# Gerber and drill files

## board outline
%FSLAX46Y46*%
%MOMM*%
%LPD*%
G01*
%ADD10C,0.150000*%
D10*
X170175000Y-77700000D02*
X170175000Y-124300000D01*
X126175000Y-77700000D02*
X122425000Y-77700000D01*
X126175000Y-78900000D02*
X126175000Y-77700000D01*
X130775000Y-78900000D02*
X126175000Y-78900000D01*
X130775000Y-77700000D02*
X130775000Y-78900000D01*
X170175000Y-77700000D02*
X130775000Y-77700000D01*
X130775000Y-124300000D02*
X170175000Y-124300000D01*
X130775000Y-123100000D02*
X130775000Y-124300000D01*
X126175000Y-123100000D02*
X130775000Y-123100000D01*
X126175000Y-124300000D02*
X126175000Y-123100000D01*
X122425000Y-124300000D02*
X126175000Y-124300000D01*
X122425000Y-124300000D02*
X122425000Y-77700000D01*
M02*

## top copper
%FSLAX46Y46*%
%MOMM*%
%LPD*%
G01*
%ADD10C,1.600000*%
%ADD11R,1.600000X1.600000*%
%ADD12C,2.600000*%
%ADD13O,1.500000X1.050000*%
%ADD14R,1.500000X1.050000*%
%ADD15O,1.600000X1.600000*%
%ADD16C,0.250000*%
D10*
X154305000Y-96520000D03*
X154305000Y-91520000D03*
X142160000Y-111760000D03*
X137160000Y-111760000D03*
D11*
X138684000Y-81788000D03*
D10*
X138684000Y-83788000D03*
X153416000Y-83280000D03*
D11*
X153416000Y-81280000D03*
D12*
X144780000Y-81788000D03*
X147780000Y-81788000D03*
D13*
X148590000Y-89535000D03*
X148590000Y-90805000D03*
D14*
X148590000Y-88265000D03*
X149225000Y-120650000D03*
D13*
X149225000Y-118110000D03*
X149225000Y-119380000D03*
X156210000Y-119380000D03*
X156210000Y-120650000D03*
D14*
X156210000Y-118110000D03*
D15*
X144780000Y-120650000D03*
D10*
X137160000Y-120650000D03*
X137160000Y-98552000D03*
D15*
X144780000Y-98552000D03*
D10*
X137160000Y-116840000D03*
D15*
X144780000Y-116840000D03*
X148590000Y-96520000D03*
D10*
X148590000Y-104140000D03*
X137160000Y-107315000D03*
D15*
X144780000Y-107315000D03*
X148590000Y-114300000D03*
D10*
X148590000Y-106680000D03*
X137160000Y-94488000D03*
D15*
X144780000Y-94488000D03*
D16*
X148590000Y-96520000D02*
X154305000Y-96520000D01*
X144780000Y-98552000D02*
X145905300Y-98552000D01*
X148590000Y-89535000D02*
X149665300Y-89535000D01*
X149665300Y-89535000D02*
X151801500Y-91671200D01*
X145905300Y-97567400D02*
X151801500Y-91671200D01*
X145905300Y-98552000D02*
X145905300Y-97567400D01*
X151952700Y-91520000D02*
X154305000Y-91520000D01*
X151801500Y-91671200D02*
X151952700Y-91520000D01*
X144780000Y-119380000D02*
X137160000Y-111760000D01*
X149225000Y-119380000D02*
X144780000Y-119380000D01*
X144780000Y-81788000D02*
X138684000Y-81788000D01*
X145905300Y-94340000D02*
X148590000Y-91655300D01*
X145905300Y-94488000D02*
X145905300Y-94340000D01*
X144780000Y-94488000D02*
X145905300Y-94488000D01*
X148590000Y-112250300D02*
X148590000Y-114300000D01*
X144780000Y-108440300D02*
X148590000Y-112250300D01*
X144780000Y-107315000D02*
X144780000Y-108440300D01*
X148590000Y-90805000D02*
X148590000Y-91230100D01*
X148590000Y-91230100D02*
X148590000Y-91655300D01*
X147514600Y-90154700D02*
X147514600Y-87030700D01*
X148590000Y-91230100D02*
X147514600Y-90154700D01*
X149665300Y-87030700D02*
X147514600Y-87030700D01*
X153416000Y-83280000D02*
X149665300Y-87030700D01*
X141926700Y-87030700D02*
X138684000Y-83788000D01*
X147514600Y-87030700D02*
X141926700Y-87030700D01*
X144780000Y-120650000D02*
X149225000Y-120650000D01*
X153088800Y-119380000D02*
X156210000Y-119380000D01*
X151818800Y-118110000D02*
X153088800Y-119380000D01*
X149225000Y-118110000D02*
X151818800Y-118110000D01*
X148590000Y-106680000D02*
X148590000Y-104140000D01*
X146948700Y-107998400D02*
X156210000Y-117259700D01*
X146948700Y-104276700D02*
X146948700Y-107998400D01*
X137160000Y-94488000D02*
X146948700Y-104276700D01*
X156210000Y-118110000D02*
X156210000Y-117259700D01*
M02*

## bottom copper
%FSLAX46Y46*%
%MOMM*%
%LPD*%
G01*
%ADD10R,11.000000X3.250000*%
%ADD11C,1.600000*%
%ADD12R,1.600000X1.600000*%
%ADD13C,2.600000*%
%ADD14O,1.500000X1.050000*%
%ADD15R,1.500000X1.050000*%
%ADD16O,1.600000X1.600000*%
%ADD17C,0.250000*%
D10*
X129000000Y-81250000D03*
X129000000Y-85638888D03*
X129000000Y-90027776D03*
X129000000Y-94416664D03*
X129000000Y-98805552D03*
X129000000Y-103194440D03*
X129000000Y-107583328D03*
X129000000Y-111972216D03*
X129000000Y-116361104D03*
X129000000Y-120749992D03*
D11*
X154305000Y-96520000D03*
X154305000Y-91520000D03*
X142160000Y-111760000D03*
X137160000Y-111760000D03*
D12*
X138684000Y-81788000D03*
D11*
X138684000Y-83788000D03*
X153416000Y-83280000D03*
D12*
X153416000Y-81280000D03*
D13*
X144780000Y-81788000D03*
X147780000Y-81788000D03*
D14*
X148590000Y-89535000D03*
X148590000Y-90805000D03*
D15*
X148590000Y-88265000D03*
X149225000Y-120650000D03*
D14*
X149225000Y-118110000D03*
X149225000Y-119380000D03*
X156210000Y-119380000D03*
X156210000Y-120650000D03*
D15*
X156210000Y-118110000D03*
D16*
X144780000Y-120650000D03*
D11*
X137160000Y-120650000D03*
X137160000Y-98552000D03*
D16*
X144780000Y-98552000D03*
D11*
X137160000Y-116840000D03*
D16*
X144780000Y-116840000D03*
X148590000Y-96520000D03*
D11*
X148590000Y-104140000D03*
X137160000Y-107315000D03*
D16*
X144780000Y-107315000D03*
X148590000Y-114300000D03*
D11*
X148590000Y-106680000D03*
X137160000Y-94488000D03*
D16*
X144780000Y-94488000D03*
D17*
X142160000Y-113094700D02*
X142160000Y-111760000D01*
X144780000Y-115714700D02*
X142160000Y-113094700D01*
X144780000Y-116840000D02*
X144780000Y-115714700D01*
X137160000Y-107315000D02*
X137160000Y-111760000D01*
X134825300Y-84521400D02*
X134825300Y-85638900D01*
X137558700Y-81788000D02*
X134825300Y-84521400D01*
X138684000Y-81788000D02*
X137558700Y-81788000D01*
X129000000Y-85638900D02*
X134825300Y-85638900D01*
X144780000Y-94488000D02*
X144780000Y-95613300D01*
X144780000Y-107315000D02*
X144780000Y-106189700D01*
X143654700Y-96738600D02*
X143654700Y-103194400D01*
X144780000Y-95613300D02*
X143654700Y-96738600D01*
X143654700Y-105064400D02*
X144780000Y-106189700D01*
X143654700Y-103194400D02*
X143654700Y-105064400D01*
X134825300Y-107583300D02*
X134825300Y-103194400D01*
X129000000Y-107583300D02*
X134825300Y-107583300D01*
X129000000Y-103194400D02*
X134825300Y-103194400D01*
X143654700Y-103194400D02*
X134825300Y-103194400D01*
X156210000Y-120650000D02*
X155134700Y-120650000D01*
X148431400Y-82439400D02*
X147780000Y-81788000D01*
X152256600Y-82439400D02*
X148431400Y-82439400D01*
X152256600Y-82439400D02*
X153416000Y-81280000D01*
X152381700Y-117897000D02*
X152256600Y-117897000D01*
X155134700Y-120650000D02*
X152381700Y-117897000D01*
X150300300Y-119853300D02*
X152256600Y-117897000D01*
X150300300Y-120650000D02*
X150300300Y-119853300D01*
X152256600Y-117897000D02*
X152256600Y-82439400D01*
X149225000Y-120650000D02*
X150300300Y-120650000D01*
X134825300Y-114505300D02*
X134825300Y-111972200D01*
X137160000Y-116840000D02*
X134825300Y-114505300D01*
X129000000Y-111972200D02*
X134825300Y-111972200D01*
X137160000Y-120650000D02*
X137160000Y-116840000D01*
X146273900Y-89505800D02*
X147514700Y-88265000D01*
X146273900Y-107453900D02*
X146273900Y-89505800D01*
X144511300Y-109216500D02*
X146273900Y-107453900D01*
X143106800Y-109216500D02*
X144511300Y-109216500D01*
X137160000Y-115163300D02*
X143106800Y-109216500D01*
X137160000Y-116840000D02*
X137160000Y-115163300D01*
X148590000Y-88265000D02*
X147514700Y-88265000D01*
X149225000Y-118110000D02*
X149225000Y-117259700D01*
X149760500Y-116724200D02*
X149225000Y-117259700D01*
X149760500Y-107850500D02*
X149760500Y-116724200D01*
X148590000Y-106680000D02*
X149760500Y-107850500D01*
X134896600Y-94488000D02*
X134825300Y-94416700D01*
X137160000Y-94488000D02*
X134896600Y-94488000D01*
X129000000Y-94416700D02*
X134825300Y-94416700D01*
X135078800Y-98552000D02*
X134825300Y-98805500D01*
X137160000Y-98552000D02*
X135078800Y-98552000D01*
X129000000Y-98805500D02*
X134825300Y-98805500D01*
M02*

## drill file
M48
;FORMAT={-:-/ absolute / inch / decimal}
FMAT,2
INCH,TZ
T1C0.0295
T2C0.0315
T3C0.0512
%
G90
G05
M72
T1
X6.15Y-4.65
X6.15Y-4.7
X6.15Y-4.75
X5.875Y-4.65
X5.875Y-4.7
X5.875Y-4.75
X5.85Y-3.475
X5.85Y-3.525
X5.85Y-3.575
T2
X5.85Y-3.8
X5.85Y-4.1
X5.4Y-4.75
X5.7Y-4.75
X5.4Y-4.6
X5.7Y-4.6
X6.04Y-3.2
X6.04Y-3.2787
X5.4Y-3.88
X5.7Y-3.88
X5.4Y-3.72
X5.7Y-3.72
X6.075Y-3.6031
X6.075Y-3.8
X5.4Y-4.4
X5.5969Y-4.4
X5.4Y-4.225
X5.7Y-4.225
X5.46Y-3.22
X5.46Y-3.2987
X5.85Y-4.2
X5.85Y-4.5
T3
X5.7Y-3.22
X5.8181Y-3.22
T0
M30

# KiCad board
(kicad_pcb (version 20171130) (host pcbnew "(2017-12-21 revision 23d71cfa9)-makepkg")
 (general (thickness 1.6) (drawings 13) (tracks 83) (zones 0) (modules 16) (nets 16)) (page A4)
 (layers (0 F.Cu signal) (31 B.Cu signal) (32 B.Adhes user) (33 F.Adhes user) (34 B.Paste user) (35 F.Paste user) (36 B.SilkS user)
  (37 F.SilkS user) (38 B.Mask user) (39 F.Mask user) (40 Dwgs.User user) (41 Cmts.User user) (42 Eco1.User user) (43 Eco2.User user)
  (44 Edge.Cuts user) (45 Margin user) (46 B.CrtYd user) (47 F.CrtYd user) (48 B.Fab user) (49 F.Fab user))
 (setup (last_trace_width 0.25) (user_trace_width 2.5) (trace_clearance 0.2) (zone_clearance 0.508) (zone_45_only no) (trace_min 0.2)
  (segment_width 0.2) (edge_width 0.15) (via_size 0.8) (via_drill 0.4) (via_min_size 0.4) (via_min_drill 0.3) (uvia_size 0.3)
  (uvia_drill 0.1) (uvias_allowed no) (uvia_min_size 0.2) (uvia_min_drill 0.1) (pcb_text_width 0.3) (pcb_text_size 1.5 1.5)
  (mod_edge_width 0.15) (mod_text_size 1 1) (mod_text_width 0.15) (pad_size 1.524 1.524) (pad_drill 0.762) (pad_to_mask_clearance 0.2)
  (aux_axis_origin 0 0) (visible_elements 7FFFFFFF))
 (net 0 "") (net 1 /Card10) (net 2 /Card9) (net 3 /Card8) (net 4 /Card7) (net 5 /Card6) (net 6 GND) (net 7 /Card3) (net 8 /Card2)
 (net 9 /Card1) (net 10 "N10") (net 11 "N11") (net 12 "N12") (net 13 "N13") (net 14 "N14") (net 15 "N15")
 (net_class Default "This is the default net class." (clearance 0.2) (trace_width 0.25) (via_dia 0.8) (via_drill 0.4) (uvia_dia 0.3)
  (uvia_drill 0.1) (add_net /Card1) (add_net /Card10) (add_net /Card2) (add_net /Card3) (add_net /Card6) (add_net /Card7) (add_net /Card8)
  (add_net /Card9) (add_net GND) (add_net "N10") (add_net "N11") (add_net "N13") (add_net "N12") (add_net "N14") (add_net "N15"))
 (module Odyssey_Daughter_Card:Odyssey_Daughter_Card (layer F.Cu) (at 129 101)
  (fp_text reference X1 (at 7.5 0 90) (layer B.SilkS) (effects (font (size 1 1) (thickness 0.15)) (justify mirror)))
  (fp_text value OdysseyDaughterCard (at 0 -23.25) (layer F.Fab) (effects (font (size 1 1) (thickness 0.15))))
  (pad 10 smd rect (at 0 -19.75) (size 11 3.25) (layers B.Cu B.Mask) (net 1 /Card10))
  (pad 9 smd rect (at 0 -15.361112) (size 11 3.25) (layers B.Cu B.Mask) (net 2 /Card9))
  (pad 8 smd rect (at 0 -10.972224) (size 11 3.25) (layers B.Cu B.Mask) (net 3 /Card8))
  (pad 7 smd rect (at 0 -6.583336) (size 11 3.25) (layers B.Cu B.Mask) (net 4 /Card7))
  (pad 6 smd rect (at 0 -2.194448) (size 11 3.25) (layers B.Cu B.Mask) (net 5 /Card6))
  (pad 5 smd rect (at 0 2.19444) (size 11 3.25) (layers B.Cu B.Mask) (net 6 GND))
  (pad 4 smd rect (at 0 6.583328) (size 11 3.25) (layers B.Cu B.Mask) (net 6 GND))
  (pad 3 smd rect (at 0 10.972216) (size 11 3.25) (layers B.Cu B.Mask) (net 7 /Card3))
  (pad 2 smd rect (at 0 15.361104) (size 11 3.25) (layers B.Cu B.Mask) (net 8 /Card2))
  (pad 1 smd rect (at 0 19.749992) (size 11 3.25) (layers B.Cu B.Mask) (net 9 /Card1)))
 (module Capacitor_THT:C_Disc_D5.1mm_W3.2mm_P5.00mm (layer F.Cu) (at 154.305 96.52 90)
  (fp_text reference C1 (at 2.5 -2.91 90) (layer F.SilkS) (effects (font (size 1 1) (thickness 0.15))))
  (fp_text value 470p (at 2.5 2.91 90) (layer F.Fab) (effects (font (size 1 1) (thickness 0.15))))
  (pad 1 thru_hole circle (at 0 0 90) (size 1.6 1.6) (drill 0.8) (layers *.Cu *.Mask) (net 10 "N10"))
  (pad 2 thru_hole circle (at 5 0 90) (size 1.6 1.6) (drill 0.8) (layers *.Cu *.Mask) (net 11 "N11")))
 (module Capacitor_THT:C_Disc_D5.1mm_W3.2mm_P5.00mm (layer F.Cu) (at 137.16 111.76)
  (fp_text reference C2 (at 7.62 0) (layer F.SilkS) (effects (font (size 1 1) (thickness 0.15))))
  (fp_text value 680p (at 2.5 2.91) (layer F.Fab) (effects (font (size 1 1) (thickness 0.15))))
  (pad 2 thru_hole circle (at 5 0) (size 1.6 1.6) (drill 0.8) (layers *.Cu *.Mask) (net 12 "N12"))
  (pad 1 thru_hole circle (at 0 0) (size 1.6 1.6) (drill 0.8) (layers *.Cu *.Mask) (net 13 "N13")))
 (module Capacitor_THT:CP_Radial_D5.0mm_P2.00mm (layer F.Cu) (at 138.684 81.788 270)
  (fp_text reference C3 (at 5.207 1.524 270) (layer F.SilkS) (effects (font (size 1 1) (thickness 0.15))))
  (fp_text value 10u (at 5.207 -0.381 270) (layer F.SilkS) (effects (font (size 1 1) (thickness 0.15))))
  (pad 1 thru_hole rect (at 0 0 270) (size 1.6 1.6) (drill 0.8) (layers *.Cu *.Mask) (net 2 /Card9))
  (pad 2 thru_hole circle (at 2 0 270) (size 1.6 1.6) (drill 0.8) (layers *.Cu *.Mask) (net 6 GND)))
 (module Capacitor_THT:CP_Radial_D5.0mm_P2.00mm (layer F.Cu) (at 153.416 81.28 270)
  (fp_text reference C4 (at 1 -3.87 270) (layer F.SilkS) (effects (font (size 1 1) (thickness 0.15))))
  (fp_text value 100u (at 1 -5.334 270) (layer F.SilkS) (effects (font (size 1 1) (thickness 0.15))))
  (pad 2 thru_hole circle (at 2 0 270) (size 1.6 1.6) (drill 0.8) (layers *.Cu *.Mask) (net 6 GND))
  (pad 1 thru_hole rect (at 0 0 270) (size 1.6 1.6) (drill 0.8) (layers *.Cu *.Mask) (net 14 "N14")))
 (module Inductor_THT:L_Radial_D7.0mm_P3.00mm (layer F.Cu) (at 144.78 81.788)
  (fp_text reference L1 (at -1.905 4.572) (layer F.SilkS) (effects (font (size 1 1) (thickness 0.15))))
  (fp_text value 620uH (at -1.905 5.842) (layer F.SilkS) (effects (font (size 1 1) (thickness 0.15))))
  (pad 1 thru_hole circle (at 0 0) (size 2.6 2.6) (drill 1.3) (layers *.Cu *.Mask) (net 2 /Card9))
  (pad 2 thru_hole circle (at 3 0) (size 2.6 2.6) (drill 1.3) (layers *.Cu *.Mask) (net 14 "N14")))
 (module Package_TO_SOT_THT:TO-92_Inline (layer F.Cu) (at 148.59 88.265 270)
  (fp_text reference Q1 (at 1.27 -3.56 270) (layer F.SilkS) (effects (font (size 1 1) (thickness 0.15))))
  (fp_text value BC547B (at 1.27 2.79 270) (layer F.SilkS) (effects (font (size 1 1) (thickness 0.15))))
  (pad 2 thru_hole oval (at 1.27 0 270) (size 1.05 1.5) (drill 0.75) (layers *.Cu *.Mask) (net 11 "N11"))
  (pad 3 thru_hole oval (at 2.54 0 270) (size 1.05 1.5) (drill 0.75) (layers *.Cu *.Mask) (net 6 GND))
  (pad 1 thru_hole rect (at 0 0 270) (size 1.05 1.5) (drill 0.75) (layers *.Cu *.Mask) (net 7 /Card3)))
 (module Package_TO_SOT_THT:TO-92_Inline (layer F.Cu) (at 149.225 120.65 90)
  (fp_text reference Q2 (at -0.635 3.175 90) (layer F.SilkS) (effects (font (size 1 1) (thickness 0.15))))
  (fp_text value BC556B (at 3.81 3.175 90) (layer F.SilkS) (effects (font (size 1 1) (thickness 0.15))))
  (pad 1 thru_hole rect (at 0 0 90) (size 1.05 1.5) (drill 0.75) (layers *.Cu *.Mask) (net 14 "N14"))
  (pad 3 thru_hole oval (at 2.54 0 90) (size 1.05 1.5) (drill 0.75) (layers *.Cu *.Mask) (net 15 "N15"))
  (pad 2 thru_hole oval (at 1.27 0 90) (size 1.05 1.5) (drill 0.75) (layers *.Cu *.Mask) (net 13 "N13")))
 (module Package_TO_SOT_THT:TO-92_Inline (layer F.Cu) (at 156.21 118.11 270)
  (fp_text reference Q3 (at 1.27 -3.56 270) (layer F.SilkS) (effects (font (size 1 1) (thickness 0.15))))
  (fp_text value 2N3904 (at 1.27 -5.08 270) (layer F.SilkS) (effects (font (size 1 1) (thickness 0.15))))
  (pad 2 thru_hole oval (at 1.27 0 270) (size 1.05 1.5) (drill 0.75) (layers *.Cu *.Mask) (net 15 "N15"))
  (pad 3 thru_hole oval (at 2.54 0 270) (size 1.05 1.5) (drill 0.75) (layers *.Cu *.Mask) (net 14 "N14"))
  (pad 1 thru_hole rect (at 0 0 270) (size 1.05 1.5) (drill 0.75) (layers *.Cu *.Mask) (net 4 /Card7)))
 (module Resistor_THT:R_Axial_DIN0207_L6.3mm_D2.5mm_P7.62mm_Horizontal (layer F.Cu) (at 137.16 120.65)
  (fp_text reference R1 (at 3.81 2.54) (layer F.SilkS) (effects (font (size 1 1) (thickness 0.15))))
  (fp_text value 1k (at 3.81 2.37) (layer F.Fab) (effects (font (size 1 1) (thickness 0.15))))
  (pad 2 thru_hole oval (at 7.62 0) (size 1.6 1.6) (drill 0.8) (layers *.Cu *.Mask) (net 14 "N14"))
  (pad 1 thru_hole circle (at 0 0) (size 1.6 1.6) (drill 0.8) (layers *.Cu *.Mask) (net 7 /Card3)))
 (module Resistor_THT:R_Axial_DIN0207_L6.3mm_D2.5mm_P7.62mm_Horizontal (layer F.Cu) (at 137.16 98.552)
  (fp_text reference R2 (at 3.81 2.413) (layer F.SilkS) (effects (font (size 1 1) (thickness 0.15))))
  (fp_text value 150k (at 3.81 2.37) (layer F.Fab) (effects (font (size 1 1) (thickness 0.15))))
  (pad 1 thru_hole circle (at 0 0) (size 1.6 1.6) (drill 0.8) (layers *.Cu *.Mask) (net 5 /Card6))
  (pad 2 thru_hole oval (at 7.62 0) (size 1.6 1.6) (drill 0.8) (layers *.Cu *.Mask) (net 11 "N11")))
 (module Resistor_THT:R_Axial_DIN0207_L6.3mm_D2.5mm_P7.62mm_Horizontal (layer F.Cu) (at 137.16 116.84)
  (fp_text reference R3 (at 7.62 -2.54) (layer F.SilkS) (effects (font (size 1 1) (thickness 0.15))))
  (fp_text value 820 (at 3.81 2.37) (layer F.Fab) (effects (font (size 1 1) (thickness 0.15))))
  (pad 1 thru_hole circle (at 0 0) (size 1.6 1.6) (drill 0.8) (layers *.Cu *.Mask) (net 7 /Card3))
  (pad 2 thru_hole oval (at 7.62 0) (size 1.6 1.6) (drill 0.8) (layers *.Cu *.Mask) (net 12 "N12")))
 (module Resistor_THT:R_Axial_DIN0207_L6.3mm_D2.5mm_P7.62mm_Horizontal (layer F.Cu) (at 148.59 104.14 90)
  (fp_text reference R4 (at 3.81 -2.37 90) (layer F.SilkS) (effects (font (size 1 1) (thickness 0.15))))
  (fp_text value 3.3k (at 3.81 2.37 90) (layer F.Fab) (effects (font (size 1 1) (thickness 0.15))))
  (pad 2 thru_hole oval (at 7.62 0 90) (size 1.6 1.6) (drill 0.8) (layers *.Cu *.Mask) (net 10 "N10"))
  (pad 1 thru_hole circle (at 0 0 90) (size 1.6 1.6) (drill 0.8) (layers *.Cu *.Mask) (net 15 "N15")))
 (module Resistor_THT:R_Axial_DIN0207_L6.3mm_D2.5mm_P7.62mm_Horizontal (layer F.Cu) (at 137.16 107.315)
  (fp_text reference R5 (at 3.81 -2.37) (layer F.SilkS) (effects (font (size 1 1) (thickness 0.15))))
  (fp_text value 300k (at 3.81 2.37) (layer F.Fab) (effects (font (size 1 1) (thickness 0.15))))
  (pad 1 thru_hole circle (at 0 0) (size 1.6 1.6) (drill 0.8) (layers *.Cu *.Mask) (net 13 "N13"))
  (pad 2 thru_hole oval (at 7.62 0) (size 1.6 1.6) (drill 0.8) (layers *.Cu *.Mask) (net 6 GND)))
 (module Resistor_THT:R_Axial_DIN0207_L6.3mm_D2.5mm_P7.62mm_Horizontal (layer F.Cu) (at 148.59 106.68 270)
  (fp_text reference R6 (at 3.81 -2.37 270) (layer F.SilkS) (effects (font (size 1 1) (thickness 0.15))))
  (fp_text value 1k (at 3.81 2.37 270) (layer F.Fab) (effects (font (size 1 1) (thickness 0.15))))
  (pad 2 thru_hole oval (at 7.62 0 270) (size 1.6 1.6) (drill 0.8) (layers *.Cu *.Mask) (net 6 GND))
  (pad 1 thru_hole circle (at 0 0 270) (size 1.6 1.6) (drill 0.8) (layers *.Cu *.Mask) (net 15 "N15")))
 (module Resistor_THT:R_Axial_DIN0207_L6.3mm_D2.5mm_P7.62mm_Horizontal (layer F.Cu) (at 137.16 94.488)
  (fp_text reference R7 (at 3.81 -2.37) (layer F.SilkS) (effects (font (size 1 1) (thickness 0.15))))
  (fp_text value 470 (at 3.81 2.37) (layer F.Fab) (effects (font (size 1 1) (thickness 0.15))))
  (pad 1 thru_hole circle (at 0 0) (size 1.6 1.6) (drill 0.8) (layers *.Cu *.Mask) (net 4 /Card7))
  (pad 2 thru_hole oval (at 7.62 0) (size 1.6 1.6) (drill 0.8) (layers *.Cu *.Mask) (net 6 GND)))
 (gr_line (start 170.175 77.7) (end 170.175 124.3) (layer Edge.Cuts) (width 0.15))
 (gr_line (start 126.175 77.7) (end 122.425 77.7) (layer Edge.Cuts) (width 0.15))
 (gr_line (start 126.175 78.9) (end 126.175 77.7) (layer Edge.Cuts) (width 0.15))
 (gr_line (start 130.775 78.9) (end 126.175 78.9) (layer Edge.Cuts) (width 0.15))
 (gr_line (start 130.775 77.7) (end 130.775 78.9) (layer Edge.Cuts) (width 0.15))
 (gr_line (start 170.175 77.7) (end 130.775 77.7) (layer Edge.Cuts) (width 0.15))
 (gr_line (start 130.775 124.3) (end 170.175 124.3) (layer Edge.Cuts) (width 0.15))
 (gr_line (start 130.775 123.1) (end 130.775 124.3) (layer Edge.Cuts) (width 0.15))
 (gr_line (start 126.175 123.1) (end 130.775 123.1) (layer Edge.Cuts) (width 0.15))
 (gr_line (start 126.175 124.3) (end 126.175 123.1) (layer Edge.Cuts) (width 0.15))
 (gr_line (start 122.425 124.3) (end 126.175 124.3) (layer Edge.Cuts) (width 0.15))
 (gr_line (start 122.425 124.3) (end 122.425 77.7) (layer Edge.Cuts) (width 0.15))
 (segment (start 148.59 96.52) (end 154.305 96.52) (width 0.25) (layer F.Cu) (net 10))
 (segment (start 144.78 98.552) (end 145.9053 98.552) (width 0.25) (layer F.Cu) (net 11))
 (segment (start 148.59 89.535) (end 149.6653 89.535) (width 0.25) (layer F.Cu) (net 11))
 (segment (start 149.6653 89.535) (end 151.8015 91.6712) (width 0.25) (layer F.Cu) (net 11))
 (segment (start 145.9053 97.5674) (end 151.8015 91.6712) (width 0.25) (layer F.Cu) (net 11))
 (segment (start 145.9053 98.552) (end 145.9053 97.5674) (width 0.25) (layer F.Cu) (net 11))
 (segment (start 151.9527 91.52) (end 154.305 91.52) (width 0.25) (layer F.Cu) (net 11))
 (segment (start 151.8015 91.6712) (end 151.9527 91.52) (width 0.25) (layer F.Cu) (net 11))
 (segment (start 142.16 113.0947) (end 142.16 111.76) (width 0.25) (layer B.Cu) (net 12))
 (segment (start 144.78 115.7147) (end 142.16 113.0947) (width 0.25) (layer B.Cu) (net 12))
 (segment (start 144.78 116.84) (end 144.78 115.7147) (width 0.25) (layer B.Cu) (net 12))
 (segment (start 137.16 107.315) (end 137.16 111.76) (width 0.25) (layer B.Cu) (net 13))
 (segment (start 144.78 119.38) (end 137.16 111.76) (width 0.25) (layer F.Cu) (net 13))
 (segment (start 149.225 119.38) (end 144.78 119.38) (width 0.25) (layer F.Cu) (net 13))
 (segment (start 144.78 81.788) (end 138.684 81.788) (width 0.25) (layer F.Cu) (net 2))
 (segment (start 134.8253 84.5214) (end 134.8253 85.6389) (width 0.25) (layer B.Cu) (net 2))
 (segment (start 137.5587 81.788) (end 134.8253 84.5214) (width 0.25) (layer B.Cu) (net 2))
 (segment (start 138.684 81.788) (end 137.5587 81.788) (width 0.25) (layer B.Cu) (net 2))
 (segment (start 129 85.6389) (end 134.8253 85.6389) (width 0.25) (layer B.Cu) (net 2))
 (segment (start 145.9053 94.34) (end 148.59 91.6553) (width 0.25) (layer F.Cu) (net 6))
 (segment (start 145.9053 94.488) (end 145.9053 94.34) (width 0.25) (layer F.Cu) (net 6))
 (segment (start 144.78 94.488) (end 145.9053 94.488) (width 0.25) (layer F.Cu) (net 6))
 (segment (start 148.59 112.2503) (end 148.59 114.3) (width 0.25) (layer F.Cu) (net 6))
 (segment (start 144.78 108.4403) (end 148.59 112.2503) (width 0.25) (layer F.Cu) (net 6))
 (segment (start 144.78 107.315) (end 144.78 108.4403) (width 0.25) (layer F.Cu) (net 6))
 (segment (start 144.78 94.488) (end 144.78 95.6133) (width 0.25) (layer B.Cu) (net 6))
 (segment (start 144.78 107.315) (end 144.78 106.1897) (width 0.25) (layer B.Cu) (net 6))
 (segment (start 143.6547 96.7386) (end 143.6547 103.1944) (width 0.25) (layer B.Cu) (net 6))
 (segment (start 144.78 95.6133) (end 143.6547 96.7386) (width 0.25) (layer B.Cu) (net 6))
 (segment (start 143.6547 105.0644) (end 144.78 106.1897) (width 0.25) (layer B.Cu) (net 6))
 (segment (start 143.6547 103.1944) (end 143.6547 105.0644) (width 0.25) (layer B.Cu) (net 6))
 (segment (start 134.8253 107.5833) (end 134.8253 103.1944) (width 0.25) (layer B.Cu) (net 6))
 (segment (start 129 107.5833) (end 134.8253 107.5833) (width 0.25) (layer B.Cu) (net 6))
 (segment (start 129 103.1944) (end 134.8253 103.1944) (width 0.25) (layer B.Cu) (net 6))
 (segment (start 143.6547 103.1944) (end 134.8253 103.1944) (width 0.25) (layer B.Cu) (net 6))
 (segment (start 148.59 90.805) (end 148.59 91.2301) (width 0.25) (layer F.Cu) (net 6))
 (segment (start 148.59 91.2301) (end 148.59 91.6553) (width 0.25) (layer F.Cu) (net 6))
 (segment (start 147.5146 90.1547) (end 147.5146 87.0307) (width 0.25) (layer F.Cu) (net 6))
 (segment (start 148.59 91.2301) (end 147.5146 90.1547) (width 0.25) (layer F.Cu) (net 6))
 (segment (start 149.6653 87.0307) (end 147.5146 87.0307) (width 0.25) (layer F.Cu) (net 6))
 (segment (start 153.416 83.28) (end 149.6653 87.0307) (width 0.25) (layer F.Cu) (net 6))
 (segment (start 141.9267 87.0307) (end 138.684 83.788) (width 0.25) (layer F.Cu) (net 6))
 (segment (start 147.5146 87.0307) (end 141.9267 87.0307) (width 0.25) (layer F.Cu) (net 6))
 (segment (start 144.78 120.65) (end 149.225 120.65) (width 0.25) (layer F.Cu) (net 14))
 (segment (start 156.21 120.65) (end 155.1347 120.65) (width 0.25) (layer B.Cu) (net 14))
 (segment (start 148.4314 82.4394) (end 147.78 81.788) (width 0.25) (layer B.Cu) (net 14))
 (segment (start 152.2566 82.4394) (end 148.4314 82.4394) (width 0.25) (layer B.Cu) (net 14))
 (segment (start 152.2566 82.4394) (end 153.416 81.28) (width 0.25) (layer B.Cu) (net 14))
 (segment (start 152.3817 117.897) (end 152.2566 117.897) (width 0.25) (layer B.Cu) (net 14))
 (segment (start 155.1347 120.65) (end 152.3817 117.897) (width 0.25) (layer B.Cu) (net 14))
 (segment (start 150.3003 119.8533) (end 152.2566 117.897) (width 0.25) (layer B.Cu) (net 14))
 (segment (start 150.3003 120.65) (end 150.3003 119.8533) (width 0.25) (layer B.Cu) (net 14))
 (segment (start 152.2566 117.897) (end 152.2566 82.4394) (width 0.25) (layer B.Cu) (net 14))
 (segment (start 149.225 120.65) (end 150.3003 120.65) (width 0.25) (layer B.Cu) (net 14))
 (segment (start 134.8253 114.5053) (end 134.8253 111.9722) (width 0.25) (layer B.Cu) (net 7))
 (segment (start 137.16 116.84) (end 134.8253 114.5053) (width 0.25) (layer B.Cu) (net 7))
 (segment (start 129 111.9722) (end 134.8253 111.9722) (width 0.25) (layer B.Cu) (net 7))
 (segment (start 137.16 120.65) (end 137.16 116.84) (width 0.25) (layer B.Cu) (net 7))
 (segment (start 146.2739 89.5058) (end 147.5147 88.265) (width 0.25) (layer B.Cu) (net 7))
 (segment (start 146.2739 107.4539) (end 146.2739 89.5058) (width 0.25) (layer B.Cu) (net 7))
 (segment (start 144.5113 109.2165) (end 146.2739 107.4539) (width 0.25) (layer B.Cu) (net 7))
 (segment (start 143.1068 109.2165) (end 144.5113 109.2165) (width 0.25) (layer B.Cu) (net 7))
 (segment (start 137.16 115.1633) (end 143.1068 109.2165) (width 0.25) (layer B.Cu) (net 7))
 (segment (start 137.16 116.84) (end 137.16 115.1633) (width 0.25) (layer B.Cu) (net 7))
 (segment (start 148.59 88.265) (end 147.5147 88.265) (width 0.25) (layer B.Cu) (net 7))
 (segment (start 149.225 118.11) (end 149.225 117.2597) (width 0.25) (layer B.Cu) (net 15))
 (segment (start 149.7605 116.7242) (end 149.225 117.2597) (width 0.25) (layer B.Cu) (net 15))
 (segment (start 149.7605 107.8505) (end 149.7605 116.7242) (width 0.25) (layer B.Cu) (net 15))
 (segment (start 148.59 106.68) (end 149.7605 107.8505) (width 0.25) (layer B.Cu) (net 15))
 (segment (start 153.0888 119.38) (end 156.21 119.38) (width 0.25) (layer F.Cu) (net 15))
 (segment (start 151.8188 118.11) (end 153.0888 119.38) (width 0.25) (layer F.Cu) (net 15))
 (segment (start 149.225 118.11) (end 151.8188 118.11) (width 0.25) (layer F.Cu) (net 15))
 (segment (start 148.59 106.68) (end 148.59 104.14) (width 0.25) (layer F.Cu) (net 15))
 (segment (start 134.8966 94.488) (end 134.8253 94.4167) (width 0.25) (layer B.Cu) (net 4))
 (segment (start 137.16 94.488) (end 134.8966 94.488) (width 0.25) (layer B.Cu) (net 4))
 (segment (start 129 94.4167) (end 134.8253 94.4167) (width 0.25) (layer B.Cu) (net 4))
 (segment (start 146.9487 107.9984) (end 156.21 117.2597) (width 0.25) (layer F.Cu) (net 4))
 (segment (start 146.9487 104.2767) (end 146.9487 107.9984) (width 0.25) (layer F.Cu) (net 4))
 (segment (start 137.16 94.488) (end 146.9487 104.2767) (width 0.25) (layer F.Cu) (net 4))
 (segment (start 156.21 118.11) (end 156.21 117.2597) (width 0.25) (layer F.Cu) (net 4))
 (segment (start 135.0788 98.552) (end 134.8253 98.8055) (width 0.25) (layer B.Cu) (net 5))
 (segment (start 137.16 98.552) (end 135.0788 98.552) (width 0.25) (layer B.Cu) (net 5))
 (segment (start 129 98.8055) (end 134.8253 98.8055) (width 0.25) (layer B.Cu) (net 5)))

